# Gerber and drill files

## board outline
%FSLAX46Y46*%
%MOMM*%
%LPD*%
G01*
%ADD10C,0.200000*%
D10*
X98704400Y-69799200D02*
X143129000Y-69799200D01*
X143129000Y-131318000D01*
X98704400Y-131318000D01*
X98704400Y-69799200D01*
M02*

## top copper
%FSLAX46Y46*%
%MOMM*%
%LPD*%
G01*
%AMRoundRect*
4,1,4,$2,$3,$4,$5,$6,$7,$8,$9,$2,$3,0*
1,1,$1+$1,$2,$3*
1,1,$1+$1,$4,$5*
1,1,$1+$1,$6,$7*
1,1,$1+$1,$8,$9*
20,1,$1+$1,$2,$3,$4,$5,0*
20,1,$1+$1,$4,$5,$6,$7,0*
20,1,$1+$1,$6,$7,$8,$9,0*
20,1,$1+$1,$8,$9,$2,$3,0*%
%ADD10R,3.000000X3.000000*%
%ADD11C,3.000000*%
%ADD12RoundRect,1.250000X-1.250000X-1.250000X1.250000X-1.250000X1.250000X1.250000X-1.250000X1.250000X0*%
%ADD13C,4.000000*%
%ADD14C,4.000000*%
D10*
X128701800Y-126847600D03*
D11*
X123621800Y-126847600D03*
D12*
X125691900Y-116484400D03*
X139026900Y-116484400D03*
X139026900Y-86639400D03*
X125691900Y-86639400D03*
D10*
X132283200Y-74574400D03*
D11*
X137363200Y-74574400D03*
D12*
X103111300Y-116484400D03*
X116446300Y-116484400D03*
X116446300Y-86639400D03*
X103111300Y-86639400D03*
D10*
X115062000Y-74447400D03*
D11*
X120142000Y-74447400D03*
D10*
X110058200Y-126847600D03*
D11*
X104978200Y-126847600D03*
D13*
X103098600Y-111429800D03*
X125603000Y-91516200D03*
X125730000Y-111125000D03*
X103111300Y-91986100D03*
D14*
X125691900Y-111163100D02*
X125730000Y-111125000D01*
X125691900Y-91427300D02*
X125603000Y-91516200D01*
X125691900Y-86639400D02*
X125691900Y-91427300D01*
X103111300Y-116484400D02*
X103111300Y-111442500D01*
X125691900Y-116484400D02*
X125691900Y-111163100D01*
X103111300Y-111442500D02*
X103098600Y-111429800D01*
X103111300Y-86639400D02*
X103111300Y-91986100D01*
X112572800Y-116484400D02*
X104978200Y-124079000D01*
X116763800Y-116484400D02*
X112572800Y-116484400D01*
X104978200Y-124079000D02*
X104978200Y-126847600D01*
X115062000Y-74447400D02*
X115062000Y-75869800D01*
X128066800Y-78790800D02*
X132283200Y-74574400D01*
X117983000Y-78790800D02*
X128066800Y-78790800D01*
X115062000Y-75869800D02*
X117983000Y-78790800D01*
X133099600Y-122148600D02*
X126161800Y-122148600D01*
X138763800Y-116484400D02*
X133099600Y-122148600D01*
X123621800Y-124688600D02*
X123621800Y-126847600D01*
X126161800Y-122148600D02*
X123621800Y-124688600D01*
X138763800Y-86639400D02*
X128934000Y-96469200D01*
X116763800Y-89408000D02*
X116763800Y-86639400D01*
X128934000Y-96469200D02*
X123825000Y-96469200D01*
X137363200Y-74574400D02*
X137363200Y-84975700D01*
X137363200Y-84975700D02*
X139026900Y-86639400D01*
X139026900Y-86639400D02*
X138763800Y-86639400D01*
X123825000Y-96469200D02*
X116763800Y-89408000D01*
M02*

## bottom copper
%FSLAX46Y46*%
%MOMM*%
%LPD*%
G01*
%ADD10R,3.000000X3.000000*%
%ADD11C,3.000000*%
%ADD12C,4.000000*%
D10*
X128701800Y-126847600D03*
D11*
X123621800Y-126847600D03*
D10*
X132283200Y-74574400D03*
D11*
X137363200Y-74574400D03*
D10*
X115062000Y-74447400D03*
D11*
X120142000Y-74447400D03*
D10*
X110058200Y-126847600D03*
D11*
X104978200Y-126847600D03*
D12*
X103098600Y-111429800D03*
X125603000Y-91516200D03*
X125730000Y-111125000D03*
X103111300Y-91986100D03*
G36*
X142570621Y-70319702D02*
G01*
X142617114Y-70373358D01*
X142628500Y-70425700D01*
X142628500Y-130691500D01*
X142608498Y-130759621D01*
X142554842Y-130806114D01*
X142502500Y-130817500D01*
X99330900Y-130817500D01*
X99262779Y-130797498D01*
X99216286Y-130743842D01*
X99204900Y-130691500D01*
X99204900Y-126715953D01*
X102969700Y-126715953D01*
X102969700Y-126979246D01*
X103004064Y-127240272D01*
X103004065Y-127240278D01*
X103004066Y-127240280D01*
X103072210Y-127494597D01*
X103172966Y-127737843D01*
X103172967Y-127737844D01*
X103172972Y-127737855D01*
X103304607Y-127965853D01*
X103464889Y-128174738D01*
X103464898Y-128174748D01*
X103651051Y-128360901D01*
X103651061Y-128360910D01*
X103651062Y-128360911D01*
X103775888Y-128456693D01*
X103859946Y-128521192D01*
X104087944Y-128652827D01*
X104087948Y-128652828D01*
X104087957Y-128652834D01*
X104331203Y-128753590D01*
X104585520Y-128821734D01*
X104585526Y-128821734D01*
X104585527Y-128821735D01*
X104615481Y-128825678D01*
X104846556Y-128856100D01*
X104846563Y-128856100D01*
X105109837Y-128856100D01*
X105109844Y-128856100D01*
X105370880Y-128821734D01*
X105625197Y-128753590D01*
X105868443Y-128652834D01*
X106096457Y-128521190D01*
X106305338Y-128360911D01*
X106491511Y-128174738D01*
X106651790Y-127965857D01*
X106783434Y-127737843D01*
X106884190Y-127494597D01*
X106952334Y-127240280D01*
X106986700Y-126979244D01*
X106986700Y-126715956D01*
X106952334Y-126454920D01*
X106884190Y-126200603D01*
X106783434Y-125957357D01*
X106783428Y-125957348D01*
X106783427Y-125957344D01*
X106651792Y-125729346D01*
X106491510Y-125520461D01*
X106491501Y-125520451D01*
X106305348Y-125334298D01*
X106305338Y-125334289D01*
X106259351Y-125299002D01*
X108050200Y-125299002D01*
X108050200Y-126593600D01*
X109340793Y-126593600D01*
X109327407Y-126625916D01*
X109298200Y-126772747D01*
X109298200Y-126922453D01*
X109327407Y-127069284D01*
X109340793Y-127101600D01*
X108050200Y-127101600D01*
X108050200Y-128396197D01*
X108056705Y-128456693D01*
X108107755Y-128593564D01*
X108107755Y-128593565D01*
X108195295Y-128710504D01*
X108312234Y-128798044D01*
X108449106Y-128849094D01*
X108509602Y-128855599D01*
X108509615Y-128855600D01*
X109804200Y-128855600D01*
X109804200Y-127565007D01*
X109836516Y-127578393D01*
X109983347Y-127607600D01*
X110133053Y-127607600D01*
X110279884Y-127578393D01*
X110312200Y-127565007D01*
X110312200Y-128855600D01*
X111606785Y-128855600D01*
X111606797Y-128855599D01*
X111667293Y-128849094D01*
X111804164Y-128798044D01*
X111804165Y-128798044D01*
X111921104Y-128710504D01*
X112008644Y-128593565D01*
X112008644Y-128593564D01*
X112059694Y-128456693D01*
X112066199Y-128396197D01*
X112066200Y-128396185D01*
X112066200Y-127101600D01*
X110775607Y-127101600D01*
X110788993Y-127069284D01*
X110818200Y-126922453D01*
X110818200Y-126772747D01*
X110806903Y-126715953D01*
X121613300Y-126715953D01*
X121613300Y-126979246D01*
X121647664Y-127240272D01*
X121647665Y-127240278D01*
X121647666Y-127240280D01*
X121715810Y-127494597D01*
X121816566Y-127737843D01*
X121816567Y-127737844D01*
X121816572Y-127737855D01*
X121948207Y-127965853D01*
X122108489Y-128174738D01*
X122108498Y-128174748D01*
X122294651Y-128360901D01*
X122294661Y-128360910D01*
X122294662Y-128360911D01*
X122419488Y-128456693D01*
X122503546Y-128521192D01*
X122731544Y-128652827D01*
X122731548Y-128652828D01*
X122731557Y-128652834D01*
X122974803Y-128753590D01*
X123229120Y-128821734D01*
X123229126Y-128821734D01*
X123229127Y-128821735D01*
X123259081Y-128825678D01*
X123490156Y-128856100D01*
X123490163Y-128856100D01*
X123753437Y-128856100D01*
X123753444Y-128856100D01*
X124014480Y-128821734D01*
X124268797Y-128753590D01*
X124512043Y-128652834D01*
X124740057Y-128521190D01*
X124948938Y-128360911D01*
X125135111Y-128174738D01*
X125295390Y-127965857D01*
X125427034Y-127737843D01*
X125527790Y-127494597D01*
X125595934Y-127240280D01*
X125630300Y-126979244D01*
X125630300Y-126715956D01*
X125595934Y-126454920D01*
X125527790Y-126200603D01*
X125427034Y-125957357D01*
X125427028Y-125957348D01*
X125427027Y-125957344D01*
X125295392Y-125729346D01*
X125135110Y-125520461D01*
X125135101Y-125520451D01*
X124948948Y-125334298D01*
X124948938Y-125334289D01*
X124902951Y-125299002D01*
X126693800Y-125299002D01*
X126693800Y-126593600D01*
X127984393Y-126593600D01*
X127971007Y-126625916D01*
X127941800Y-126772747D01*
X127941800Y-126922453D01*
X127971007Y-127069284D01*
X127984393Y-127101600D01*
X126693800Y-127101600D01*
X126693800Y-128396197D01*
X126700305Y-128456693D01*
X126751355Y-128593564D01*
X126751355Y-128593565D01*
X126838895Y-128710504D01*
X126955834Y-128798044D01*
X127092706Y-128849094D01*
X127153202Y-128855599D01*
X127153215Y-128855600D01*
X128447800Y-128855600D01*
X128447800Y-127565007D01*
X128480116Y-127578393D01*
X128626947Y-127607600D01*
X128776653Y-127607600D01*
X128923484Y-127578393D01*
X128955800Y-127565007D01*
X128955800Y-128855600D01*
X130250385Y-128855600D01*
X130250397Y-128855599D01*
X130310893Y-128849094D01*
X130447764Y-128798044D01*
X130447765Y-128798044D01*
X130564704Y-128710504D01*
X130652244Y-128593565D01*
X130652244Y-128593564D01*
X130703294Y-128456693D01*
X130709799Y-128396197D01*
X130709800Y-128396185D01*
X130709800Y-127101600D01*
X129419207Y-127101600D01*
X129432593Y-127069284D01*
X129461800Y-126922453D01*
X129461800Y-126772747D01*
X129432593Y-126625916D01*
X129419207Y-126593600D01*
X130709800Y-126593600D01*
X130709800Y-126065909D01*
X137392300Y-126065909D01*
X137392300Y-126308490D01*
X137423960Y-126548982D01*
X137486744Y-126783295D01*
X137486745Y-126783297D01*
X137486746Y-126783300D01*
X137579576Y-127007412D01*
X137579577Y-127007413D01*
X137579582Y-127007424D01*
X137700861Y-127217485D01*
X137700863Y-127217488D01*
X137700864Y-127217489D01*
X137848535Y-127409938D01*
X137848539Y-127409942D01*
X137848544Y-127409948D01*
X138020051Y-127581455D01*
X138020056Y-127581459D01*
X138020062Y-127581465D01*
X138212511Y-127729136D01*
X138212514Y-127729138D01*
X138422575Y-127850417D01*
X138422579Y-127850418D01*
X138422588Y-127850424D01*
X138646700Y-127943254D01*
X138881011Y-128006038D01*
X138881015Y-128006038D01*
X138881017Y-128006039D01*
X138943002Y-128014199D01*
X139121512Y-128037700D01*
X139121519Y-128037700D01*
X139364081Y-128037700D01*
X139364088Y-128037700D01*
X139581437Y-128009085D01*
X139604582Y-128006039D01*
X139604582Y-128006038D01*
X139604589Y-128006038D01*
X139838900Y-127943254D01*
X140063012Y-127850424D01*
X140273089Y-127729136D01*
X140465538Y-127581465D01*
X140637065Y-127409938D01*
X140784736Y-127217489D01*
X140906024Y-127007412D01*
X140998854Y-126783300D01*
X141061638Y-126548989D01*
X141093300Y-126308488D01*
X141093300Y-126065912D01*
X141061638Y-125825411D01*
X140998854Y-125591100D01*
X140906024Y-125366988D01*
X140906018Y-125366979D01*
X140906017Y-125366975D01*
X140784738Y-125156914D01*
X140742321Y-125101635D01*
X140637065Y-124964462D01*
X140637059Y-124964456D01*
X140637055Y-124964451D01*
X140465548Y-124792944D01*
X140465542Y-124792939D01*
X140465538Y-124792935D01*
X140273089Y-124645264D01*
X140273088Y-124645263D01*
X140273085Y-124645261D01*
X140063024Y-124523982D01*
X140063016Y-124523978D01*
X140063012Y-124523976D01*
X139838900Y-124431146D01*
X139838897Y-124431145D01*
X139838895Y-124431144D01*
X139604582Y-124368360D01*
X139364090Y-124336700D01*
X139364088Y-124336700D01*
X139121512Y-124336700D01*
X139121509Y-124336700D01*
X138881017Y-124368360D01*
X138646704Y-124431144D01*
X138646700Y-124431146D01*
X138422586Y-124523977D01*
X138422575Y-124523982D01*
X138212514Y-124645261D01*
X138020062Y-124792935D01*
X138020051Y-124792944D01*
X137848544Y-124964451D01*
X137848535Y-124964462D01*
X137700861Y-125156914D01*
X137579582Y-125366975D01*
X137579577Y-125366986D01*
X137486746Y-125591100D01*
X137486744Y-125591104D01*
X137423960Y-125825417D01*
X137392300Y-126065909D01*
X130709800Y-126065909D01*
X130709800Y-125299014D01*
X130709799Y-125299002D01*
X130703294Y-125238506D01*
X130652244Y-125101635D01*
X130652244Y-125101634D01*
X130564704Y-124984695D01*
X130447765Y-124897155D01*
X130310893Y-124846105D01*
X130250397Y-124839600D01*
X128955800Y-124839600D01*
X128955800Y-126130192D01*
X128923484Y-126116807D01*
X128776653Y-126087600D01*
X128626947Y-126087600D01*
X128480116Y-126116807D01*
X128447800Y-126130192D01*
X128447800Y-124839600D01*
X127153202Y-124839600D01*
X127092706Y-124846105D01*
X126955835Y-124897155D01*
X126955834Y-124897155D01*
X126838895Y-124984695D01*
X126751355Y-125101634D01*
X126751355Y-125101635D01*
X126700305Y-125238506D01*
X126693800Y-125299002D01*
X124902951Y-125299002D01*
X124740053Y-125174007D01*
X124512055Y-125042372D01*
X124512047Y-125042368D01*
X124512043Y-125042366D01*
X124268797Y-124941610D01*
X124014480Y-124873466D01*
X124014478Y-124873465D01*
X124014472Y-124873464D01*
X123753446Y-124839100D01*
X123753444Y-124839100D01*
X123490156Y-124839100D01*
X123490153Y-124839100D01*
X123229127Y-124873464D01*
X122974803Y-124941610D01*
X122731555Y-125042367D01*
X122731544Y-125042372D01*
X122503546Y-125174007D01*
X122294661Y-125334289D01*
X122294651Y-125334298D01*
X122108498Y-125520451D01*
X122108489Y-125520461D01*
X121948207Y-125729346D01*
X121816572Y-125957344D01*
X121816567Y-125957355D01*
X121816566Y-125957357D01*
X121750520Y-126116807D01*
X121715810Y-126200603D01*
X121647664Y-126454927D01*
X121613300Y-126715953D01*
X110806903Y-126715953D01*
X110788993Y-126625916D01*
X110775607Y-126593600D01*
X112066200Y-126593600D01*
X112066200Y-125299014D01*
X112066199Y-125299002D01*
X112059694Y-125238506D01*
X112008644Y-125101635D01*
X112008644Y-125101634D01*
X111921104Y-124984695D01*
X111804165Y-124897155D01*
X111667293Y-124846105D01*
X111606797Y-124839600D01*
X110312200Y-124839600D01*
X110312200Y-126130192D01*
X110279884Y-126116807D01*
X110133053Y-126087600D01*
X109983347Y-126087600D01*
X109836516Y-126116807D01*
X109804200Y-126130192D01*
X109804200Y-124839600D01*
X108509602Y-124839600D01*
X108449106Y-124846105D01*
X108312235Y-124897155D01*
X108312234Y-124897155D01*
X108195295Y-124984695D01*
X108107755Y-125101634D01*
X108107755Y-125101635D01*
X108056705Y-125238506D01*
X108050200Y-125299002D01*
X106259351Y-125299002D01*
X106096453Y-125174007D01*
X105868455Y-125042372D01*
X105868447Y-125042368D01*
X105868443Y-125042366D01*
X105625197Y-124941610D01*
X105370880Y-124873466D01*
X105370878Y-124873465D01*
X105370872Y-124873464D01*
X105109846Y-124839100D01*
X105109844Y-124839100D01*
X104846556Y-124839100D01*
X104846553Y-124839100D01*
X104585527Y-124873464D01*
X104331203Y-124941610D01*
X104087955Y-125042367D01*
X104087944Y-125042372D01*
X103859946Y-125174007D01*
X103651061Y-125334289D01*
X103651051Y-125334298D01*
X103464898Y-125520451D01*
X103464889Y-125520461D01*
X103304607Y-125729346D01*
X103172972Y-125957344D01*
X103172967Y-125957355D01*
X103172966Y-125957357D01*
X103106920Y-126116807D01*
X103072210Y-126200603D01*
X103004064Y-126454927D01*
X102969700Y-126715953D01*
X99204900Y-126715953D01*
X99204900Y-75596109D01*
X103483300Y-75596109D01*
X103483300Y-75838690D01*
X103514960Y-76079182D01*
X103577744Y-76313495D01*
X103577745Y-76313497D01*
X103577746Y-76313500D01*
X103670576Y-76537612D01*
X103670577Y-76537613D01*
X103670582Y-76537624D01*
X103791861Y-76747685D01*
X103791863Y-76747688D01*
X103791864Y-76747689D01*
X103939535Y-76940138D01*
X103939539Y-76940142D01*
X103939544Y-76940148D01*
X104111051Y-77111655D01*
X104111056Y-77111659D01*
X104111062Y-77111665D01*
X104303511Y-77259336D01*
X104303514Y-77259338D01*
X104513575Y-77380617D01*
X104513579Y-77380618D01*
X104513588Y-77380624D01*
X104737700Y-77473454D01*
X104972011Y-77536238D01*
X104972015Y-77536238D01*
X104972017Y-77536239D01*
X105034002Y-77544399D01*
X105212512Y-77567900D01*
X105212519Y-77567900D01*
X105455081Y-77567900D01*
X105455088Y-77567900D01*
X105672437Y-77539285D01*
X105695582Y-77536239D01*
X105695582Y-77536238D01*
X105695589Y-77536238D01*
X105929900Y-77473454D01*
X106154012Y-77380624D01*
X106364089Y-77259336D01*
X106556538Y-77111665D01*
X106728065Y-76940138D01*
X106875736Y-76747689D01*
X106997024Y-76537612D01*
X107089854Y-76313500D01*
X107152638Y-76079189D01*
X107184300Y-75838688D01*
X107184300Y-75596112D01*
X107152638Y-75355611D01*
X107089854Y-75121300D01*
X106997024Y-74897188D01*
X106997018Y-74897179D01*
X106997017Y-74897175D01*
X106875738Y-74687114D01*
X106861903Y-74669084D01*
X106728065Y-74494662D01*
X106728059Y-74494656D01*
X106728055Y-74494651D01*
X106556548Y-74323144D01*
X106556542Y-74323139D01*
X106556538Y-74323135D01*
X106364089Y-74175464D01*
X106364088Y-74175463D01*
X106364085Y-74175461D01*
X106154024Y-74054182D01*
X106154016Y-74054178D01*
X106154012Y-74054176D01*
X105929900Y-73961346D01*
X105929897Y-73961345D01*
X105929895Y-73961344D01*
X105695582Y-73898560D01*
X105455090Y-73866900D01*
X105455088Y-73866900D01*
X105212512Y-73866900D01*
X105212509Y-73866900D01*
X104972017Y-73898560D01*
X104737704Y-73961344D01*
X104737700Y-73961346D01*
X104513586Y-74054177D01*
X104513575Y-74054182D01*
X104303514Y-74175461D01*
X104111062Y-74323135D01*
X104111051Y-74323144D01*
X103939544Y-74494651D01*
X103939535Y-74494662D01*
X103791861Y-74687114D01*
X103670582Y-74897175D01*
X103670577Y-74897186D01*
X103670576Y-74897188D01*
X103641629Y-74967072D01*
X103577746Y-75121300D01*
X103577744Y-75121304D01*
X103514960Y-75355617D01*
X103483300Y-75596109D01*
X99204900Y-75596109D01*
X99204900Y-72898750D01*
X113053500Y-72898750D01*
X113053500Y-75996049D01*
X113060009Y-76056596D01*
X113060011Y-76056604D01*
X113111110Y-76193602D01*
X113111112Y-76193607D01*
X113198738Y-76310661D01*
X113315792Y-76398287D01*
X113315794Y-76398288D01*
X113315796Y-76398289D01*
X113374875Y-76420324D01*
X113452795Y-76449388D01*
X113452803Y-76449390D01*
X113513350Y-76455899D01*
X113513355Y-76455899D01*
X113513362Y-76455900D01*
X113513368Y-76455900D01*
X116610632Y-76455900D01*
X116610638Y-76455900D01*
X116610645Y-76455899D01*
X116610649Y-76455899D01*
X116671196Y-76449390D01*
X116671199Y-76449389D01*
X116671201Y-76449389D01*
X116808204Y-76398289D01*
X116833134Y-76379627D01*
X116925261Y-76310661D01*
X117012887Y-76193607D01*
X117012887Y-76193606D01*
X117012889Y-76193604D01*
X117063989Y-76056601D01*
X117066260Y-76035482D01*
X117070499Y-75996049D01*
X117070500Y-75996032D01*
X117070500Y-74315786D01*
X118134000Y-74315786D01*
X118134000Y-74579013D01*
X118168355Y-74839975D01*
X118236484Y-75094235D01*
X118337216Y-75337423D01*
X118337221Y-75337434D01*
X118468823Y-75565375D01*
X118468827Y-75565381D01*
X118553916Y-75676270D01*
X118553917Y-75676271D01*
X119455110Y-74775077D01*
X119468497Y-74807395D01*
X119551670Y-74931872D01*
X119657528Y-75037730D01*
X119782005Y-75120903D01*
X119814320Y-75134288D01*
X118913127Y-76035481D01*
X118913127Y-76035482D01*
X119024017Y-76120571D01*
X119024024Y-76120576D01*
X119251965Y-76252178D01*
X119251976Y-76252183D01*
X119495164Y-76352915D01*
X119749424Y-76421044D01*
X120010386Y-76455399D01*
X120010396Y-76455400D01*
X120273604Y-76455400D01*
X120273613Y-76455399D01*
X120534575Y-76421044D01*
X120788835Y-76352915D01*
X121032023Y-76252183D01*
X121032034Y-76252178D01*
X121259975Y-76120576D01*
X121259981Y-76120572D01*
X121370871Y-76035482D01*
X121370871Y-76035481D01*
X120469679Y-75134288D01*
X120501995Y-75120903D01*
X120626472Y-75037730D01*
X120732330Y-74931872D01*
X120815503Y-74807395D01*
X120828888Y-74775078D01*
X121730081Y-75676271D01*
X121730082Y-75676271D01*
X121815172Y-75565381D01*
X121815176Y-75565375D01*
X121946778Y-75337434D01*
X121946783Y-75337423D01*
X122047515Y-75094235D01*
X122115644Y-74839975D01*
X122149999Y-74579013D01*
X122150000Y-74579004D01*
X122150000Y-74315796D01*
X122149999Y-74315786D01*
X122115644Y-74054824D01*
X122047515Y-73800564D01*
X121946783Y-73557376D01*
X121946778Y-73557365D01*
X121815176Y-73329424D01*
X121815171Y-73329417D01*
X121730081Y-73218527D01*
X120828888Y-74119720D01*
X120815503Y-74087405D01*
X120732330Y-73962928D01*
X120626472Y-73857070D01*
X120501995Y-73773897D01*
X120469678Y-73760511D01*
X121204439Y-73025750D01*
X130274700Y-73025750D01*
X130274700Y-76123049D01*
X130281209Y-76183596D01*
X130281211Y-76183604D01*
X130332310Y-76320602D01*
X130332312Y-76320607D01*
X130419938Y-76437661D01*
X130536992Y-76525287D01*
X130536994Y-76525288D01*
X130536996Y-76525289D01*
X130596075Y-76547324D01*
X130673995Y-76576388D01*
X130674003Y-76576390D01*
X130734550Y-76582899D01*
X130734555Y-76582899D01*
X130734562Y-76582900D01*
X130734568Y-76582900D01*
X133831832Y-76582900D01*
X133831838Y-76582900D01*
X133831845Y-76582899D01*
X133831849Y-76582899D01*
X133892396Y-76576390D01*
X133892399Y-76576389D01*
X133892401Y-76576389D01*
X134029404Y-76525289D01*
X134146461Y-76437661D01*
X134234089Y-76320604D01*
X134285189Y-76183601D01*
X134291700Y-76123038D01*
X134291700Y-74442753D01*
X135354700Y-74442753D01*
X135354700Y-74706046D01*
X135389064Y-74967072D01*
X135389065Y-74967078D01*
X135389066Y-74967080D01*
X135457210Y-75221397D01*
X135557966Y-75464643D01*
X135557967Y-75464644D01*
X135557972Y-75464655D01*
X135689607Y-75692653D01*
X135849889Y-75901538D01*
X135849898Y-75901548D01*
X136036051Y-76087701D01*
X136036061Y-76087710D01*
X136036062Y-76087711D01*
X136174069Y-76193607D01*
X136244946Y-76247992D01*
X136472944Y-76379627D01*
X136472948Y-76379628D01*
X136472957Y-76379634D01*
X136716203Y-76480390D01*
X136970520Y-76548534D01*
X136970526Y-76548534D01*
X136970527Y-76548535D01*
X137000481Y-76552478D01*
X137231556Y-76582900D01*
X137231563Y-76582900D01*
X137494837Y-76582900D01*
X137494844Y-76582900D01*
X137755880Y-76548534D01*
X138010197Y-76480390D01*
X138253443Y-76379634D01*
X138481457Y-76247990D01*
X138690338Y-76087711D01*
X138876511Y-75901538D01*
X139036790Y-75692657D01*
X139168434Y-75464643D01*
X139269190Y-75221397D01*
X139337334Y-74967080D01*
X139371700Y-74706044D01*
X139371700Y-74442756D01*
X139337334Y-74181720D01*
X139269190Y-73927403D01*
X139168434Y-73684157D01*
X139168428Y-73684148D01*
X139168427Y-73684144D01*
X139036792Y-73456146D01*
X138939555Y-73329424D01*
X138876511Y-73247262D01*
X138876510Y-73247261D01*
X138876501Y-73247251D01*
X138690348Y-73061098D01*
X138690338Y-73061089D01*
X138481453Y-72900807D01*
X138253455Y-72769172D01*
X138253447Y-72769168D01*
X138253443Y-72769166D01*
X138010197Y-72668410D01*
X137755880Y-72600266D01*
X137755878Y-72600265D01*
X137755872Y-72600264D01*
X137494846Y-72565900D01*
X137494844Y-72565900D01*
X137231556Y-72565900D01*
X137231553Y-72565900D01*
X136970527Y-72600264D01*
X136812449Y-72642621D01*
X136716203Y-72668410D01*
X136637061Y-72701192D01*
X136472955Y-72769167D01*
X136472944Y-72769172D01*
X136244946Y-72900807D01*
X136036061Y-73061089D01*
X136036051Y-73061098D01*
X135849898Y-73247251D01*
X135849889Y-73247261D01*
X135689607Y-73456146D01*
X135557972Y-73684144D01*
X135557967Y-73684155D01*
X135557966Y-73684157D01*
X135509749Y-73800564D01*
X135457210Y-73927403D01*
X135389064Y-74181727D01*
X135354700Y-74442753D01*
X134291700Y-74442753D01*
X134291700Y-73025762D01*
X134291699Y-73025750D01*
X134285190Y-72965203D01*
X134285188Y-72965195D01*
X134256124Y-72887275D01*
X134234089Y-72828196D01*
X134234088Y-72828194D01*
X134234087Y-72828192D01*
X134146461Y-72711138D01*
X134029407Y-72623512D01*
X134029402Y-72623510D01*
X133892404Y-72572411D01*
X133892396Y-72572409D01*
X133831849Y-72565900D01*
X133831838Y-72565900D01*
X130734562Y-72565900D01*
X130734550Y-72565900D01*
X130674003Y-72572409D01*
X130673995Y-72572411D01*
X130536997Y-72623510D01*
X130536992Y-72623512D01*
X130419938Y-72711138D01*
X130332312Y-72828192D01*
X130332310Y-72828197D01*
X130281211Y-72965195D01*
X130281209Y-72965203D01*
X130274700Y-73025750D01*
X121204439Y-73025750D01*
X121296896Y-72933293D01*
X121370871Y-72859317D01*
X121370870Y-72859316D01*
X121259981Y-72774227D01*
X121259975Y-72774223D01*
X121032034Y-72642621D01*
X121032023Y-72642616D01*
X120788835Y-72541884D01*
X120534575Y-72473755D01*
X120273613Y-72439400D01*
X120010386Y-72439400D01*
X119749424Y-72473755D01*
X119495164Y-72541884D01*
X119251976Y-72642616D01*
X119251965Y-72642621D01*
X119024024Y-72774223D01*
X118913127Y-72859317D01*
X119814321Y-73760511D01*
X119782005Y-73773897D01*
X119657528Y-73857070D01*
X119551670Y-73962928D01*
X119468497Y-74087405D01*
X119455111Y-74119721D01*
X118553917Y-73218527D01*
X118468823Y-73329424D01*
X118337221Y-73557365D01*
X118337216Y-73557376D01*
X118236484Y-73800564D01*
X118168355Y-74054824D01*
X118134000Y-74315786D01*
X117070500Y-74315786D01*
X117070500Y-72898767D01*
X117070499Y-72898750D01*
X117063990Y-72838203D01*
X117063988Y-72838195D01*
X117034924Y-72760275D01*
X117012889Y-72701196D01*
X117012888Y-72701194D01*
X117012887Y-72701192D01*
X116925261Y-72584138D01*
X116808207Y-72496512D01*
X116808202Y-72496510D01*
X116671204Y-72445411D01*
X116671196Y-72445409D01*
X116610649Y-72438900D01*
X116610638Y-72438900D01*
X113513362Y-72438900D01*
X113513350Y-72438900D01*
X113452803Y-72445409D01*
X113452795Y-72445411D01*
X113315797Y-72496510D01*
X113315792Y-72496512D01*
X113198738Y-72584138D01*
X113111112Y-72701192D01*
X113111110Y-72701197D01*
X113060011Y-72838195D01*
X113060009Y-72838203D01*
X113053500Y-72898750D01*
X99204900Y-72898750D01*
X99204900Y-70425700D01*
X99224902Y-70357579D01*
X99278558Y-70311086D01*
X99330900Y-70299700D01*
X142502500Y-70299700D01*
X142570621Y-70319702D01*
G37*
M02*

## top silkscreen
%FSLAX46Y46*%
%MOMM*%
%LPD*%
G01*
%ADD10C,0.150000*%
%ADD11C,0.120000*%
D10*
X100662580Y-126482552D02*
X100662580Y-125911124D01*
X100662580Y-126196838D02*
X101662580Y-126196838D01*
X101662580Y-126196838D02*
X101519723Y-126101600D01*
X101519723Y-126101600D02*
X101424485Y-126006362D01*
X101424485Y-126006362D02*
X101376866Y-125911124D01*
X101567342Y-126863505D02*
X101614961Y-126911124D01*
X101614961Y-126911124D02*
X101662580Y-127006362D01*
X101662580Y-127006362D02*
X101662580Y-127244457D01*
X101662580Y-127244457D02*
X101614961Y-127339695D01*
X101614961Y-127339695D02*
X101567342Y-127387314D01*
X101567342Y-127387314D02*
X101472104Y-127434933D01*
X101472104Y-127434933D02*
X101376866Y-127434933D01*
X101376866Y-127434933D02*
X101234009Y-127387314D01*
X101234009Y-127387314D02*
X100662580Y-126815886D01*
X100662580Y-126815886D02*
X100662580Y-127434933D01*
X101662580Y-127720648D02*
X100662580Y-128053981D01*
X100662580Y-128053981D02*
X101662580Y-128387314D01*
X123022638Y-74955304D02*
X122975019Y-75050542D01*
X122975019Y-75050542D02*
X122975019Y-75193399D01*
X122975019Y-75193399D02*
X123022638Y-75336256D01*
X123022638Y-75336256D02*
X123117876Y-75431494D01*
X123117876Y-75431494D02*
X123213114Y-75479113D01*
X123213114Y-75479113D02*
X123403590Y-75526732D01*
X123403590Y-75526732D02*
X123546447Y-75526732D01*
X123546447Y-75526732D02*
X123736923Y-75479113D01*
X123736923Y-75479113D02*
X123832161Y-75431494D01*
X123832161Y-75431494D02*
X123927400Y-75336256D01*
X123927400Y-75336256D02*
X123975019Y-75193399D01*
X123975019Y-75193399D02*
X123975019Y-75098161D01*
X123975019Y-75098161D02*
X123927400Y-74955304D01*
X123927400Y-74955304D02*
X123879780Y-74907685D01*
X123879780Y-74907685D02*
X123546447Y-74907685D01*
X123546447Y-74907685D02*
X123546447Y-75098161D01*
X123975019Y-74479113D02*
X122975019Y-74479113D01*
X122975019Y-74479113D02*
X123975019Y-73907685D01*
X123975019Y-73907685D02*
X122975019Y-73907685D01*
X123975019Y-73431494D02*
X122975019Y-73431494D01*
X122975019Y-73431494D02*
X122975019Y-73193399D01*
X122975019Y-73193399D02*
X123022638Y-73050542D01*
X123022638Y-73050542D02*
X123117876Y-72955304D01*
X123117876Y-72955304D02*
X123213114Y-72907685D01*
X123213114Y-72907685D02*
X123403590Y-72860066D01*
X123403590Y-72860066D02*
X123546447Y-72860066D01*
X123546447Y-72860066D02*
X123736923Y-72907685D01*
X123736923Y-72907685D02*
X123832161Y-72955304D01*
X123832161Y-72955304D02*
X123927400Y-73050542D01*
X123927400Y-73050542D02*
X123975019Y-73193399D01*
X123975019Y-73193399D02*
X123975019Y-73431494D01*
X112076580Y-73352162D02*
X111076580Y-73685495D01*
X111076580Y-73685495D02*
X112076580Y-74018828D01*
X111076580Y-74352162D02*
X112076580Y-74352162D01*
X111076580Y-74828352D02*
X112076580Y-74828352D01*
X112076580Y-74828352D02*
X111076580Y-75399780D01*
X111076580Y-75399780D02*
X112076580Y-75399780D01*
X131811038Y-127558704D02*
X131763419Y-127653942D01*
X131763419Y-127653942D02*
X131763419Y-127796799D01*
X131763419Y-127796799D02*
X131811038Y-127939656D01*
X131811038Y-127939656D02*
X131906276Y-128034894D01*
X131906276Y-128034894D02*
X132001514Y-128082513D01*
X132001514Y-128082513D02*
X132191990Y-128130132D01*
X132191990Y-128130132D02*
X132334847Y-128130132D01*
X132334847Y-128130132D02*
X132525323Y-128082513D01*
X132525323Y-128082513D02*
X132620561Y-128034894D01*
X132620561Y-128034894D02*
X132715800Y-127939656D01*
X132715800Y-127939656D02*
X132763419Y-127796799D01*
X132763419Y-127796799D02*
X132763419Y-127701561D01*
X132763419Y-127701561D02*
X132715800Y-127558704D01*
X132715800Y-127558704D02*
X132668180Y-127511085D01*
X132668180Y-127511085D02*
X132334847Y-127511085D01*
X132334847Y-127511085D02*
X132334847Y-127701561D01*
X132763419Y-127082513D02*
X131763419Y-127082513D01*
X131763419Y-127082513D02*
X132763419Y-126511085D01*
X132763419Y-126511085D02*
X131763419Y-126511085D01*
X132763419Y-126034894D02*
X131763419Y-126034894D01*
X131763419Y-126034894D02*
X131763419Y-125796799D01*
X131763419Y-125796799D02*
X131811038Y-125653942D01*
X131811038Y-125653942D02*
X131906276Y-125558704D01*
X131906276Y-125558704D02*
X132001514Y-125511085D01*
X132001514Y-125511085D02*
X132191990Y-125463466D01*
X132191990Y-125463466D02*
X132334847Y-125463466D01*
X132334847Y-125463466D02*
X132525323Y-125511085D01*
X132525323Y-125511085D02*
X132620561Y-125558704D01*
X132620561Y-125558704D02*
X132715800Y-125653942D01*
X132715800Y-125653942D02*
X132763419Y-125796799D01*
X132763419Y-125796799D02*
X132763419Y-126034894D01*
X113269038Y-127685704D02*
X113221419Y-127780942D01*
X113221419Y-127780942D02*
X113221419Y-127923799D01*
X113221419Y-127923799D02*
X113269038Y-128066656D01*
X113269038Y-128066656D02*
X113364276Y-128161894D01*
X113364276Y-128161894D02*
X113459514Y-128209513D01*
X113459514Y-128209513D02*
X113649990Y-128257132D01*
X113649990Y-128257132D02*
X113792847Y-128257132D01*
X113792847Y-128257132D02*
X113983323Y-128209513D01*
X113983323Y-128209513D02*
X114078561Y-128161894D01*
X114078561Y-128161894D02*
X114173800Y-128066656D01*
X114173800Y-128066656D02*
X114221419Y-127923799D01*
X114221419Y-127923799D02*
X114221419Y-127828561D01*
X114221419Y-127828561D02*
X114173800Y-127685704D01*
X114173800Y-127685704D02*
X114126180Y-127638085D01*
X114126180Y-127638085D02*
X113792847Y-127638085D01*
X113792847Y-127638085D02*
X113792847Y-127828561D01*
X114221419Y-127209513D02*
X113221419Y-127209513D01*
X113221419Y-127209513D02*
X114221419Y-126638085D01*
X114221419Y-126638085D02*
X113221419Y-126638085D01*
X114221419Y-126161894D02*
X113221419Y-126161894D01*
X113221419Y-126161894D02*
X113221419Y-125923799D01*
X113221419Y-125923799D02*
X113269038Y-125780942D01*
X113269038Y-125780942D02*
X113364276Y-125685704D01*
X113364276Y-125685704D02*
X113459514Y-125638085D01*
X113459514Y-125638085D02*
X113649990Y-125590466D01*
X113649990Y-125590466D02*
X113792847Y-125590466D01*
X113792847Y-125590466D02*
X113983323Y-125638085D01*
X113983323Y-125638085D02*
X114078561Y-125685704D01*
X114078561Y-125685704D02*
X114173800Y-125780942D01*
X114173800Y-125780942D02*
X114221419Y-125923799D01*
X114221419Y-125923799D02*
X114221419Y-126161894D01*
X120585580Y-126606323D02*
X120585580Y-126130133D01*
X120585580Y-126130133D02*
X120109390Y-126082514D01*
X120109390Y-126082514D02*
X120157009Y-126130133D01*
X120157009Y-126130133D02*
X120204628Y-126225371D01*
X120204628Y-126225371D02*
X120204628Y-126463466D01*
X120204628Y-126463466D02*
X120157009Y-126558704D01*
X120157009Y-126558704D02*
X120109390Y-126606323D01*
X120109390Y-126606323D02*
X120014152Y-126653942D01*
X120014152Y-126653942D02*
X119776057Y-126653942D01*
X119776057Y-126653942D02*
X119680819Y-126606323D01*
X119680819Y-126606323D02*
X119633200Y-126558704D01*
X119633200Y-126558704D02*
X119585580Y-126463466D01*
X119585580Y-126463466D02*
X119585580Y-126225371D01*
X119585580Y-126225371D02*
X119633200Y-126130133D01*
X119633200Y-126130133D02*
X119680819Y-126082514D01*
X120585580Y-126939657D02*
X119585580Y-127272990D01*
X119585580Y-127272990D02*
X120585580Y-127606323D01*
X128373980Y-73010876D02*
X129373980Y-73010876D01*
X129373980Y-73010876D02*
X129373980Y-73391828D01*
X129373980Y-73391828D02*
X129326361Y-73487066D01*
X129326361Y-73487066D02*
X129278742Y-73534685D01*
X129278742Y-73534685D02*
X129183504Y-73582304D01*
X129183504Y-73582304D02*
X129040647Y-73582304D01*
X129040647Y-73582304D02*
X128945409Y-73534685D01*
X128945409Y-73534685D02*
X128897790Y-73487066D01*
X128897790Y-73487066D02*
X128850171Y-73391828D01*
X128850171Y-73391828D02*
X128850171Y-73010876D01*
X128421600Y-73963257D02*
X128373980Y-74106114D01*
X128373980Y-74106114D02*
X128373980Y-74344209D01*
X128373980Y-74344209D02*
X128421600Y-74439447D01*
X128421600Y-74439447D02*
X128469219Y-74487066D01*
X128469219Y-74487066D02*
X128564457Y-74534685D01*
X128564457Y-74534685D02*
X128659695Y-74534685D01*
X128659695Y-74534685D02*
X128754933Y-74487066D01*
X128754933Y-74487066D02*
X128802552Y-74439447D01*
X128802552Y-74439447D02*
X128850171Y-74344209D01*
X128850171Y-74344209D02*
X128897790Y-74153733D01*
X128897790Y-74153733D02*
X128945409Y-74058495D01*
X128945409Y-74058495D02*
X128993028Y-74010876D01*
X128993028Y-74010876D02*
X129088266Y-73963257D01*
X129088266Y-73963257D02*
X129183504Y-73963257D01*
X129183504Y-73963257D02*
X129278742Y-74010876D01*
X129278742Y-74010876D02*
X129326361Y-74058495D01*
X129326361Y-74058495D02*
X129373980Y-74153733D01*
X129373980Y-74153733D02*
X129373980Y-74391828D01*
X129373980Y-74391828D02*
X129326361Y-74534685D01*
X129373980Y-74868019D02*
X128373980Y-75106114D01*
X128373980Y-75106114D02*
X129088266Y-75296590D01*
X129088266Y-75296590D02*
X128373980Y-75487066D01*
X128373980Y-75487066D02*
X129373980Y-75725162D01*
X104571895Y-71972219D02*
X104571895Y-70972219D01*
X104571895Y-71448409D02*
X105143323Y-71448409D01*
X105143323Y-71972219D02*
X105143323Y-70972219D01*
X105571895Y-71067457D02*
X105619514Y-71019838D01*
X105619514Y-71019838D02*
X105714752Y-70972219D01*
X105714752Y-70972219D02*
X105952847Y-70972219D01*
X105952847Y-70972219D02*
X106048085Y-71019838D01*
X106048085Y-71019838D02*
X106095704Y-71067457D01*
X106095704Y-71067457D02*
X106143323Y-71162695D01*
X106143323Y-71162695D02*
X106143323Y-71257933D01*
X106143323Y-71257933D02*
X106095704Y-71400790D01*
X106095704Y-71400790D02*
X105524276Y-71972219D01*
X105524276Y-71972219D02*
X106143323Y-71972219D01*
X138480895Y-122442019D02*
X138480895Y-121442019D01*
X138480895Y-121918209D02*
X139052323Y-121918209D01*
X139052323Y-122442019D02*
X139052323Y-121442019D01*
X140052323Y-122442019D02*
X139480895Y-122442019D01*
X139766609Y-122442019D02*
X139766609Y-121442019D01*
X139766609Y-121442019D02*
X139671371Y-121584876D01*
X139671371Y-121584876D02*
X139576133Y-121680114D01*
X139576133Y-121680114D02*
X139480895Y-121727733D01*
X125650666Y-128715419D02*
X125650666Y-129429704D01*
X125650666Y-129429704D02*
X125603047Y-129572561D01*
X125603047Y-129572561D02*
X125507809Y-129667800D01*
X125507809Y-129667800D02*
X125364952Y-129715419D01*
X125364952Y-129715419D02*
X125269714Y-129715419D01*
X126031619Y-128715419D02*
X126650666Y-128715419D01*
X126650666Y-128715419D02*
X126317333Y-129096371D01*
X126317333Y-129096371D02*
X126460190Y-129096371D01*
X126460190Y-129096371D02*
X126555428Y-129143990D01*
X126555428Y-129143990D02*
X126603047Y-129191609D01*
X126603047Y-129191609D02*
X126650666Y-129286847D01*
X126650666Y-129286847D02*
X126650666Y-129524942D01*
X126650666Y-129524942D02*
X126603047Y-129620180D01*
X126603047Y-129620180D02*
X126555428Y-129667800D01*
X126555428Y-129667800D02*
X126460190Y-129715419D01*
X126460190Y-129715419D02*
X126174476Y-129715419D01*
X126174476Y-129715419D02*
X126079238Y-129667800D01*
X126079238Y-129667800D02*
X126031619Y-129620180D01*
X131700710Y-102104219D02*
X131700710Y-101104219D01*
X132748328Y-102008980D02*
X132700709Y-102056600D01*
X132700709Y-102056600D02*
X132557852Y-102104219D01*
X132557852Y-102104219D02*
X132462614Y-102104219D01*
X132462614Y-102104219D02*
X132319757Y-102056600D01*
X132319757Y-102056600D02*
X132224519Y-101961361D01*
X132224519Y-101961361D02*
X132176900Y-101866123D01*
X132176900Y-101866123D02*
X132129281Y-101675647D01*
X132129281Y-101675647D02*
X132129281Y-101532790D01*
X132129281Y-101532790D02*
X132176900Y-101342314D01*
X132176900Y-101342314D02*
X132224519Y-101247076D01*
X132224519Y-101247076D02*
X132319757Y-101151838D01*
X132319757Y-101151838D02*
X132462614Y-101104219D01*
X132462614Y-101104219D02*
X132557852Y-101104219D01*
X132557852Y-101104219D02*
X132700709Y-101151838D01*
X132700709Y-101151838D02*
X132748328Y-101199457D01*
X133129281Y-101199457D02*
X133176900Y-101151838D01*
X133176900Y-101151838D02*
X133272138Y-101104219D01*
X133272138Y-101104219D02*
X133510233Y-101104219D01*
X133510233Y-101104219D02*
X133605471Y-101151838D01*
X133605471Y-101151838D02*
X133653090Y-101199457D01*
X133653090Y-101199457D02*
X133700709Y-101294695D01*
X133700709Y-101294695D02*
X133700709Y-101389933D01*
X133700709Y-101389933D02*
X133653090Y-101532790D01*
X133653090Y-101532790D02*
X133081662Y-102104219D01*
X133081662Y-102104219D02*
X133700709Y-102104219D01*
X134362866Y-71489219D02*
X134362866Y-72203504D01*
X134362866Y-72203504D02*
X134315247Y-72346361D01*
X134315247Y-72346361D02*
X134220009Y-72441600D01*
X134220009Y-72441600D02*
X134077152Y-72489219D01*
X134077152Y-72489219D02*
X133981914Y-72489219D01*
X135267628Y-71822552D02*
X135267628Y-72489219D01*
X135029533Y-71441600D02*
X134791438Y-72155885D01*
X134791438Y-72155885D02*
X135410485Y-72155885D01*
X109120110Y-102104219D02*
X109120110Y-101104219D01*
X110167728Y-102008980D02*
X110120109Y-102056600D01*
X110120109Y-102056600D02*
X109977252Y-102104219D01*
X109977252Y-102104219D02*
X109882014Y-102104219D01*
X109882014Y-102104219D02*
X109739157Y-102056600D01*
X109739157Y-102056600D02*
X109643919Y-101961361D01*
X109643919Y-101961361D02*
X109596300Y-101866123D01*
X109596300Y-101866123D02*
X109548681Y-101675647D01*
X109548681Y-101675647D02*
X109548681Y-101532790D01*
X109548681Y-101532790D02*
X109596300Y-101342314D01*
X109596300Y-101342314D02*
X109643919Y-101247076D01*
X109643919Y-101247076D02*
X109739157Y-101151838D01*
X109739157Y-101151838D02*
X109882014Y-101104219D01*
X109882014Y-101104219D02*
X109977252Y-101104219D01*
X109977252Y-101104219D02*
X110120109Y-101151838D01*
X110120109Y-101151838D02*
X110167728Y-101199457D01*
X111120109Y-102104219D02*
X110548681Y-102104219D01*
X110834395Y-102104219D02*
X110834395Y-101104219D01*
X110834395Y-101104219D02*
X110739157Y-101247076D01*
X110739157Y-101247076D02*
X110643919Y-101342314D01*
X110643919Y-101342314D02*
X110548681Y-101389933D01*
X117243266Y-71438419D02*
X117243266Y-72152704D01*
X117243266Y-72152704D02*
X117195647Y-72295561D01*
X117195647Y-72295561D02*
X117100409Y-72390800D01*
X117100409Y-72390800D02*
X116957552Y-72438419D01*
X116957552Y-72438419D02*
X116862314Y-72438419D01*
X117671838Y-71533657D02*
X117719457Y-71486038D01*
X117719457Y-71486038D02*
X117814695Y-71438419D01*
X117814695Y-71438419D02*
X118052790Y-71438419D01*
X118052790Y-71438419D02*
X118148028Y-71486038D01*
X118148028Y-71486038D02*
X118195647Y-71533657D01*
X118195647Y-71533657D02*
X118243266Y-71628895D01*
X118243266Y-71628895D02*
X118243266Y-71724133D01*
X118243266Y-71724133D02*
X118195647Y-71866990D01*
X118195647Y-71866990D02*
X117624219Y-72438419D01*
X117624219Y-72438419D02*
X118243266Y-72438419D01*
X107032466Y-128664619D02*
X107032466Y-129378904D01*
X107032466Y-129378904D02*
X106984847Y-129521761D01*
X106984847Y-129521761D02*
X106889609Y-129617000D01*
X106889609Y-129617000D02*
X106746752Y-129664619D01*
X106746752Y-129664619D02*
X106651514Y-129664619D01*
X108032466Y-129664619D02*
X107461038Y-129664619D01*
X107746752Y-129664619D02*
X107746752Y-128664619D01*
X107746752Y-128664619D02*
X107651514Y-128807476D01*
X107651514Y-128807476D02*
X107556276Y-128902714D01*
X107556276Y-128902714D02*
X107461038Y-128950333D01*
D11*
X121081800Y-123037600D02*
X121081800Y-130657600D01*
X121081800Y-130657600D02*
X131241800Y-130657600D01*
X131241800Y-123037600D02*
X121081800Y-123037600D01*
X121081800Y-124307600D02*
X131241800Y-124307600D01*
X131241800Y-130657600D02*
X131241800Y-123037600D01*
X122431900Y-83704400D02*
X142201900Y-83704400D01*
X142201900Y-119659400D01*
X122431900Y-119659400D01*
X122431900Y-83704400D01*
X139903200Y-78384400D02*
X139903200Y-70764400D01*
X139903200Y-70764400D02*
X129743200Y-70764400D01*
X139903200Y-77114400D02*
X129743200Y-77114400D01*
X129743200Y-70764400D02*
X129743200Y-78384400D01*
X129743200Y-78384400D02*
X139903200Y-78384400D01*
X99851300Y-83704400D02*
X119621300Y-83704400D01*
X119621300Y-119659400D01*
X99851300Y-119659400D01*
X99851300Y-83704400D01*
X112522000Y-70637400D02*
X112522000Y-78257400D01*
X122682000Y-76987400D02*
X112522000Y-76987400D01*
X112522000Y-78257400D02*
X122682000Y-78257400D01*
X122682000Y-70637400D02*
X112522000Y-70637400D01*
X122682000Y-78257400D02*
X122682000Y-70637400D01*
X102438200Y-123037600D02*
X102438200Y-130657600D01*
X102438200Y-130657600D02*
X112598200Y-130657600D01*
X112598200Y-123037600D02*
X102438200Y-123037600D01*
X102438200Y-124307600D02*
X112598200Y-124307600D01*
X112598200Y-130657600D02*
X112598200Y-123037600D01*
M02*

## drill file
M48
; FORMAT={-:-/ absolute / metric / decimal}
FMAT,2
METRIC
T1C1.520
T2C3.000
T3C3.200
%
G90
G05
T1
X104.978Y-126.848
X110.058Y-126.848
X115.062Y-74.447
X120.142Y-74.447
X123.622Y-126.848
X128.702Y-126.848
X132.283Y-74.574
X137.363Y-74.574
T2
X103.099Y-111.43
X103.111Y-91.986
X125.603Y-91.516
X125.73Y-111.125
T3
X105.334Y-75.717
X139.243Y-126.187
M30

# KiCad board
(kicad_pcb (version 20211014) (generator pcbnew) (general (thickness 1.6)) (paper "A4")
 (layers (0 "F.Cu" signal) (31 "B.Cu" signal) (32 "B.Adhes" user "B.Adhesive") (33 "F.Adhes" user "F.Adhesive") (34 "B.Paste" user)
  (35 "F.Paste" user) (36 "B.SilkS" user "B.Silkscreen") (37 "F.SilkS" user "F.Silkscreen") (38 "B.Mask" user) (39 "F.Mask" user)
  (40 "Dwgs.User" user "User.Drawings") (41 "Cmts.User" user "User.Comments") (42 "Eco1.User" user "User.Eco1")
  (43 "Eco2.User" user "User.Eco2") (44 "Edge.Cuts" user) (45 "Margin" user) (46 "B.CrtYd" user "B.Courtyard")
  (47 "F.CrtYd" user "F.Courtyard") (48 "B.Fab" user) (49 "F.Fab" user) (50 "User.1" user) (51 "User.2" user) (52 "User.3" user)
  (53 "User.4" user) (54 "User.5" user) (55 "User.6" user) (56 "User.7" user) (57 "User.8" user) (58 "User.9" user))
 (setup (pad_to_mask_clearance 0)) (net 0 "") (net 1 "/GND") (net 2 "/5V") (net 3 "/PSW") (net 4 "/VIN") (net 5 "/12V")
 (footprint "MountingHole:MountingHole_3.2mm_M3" (layer "F.Cu") (at 105.3338 75.7174)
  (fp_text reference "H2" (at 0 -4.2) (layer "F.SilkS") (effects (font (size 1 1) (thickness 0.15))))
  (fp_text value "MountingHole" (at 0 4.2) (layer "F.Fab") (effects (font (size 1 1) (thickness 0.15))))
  (pad "" np_thru_hole circle (at 0 0) (size 3.2 3.2) (drill 3.2) (layers *.Cu *.Mask)))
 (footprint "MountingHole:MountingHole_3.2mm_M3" (layer "F.Cu") (at 139.2428 126.1872)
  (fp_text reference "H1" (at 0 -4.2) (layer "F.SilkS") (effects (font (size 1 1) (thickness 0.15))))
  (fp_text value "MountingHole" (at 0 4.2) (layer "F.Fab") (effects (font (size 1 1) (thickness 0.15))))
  (pad "" np_thru_hole circle (at 0 0) (size 3.2 3.2) (drill 3.2) (layers *.Cu *.Mask)))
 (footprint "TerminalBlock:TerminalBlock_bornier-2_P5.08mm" (layer "F.Cu") (at 128.7018 126.8476 180)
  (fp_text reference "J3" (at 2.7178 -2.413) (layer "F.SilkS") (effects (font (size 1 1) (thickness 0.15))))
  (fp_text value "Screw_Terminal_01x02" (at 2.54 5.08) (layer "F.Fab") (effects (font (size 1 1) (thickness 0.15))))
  (fp_line (start 7.62 3.81) (end 7.62 -3.81) (layer "F.SilkS") (width 0.12))
  (fp_line (start 7.62 -3.81) (end -2.54 -3.81) (layer "F.SilkS") (width 0.12))
  (fp_line (start -2.54 3.81) (end 7.62 3.81) (layer "F.SilkS") (width 0.12))
  (fp_line (start 7.62 2.54) (end -2.54 2.54) (layer "F.SilkS") (width 0.12))
  (fp_line (start -2.54 -3.81) (end -2.54 3.81) (layer "F.SilkS") (width 0.12))
  (pad "1" thru_hole rect (at 0 0 180) (size 3 3) (drill 1.52) (layers *.Cu *.Mask) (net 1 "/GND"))
  (pad "2" thru_hole circle (at 5.08 0 180) (size 3 3) (drill 1.52) (layers *.Cu *.Mask) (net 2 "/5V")))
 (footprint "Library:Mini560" (layer "F.Cu") (at 123.1519 86.6394)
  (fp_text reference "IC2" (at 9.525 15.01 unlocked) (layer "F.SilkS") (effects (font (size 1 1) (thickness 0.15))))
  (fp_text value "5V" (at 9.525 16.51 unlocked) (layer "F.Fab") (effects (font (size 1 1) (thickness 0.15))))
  (fp_rect (start -0.72 -2.935) (end 19.05 33.02) (layer "F.SilkS") (width 0.12) (fill none))
  (pad "1" smd roundrect (at 2.54 29.845) (size 5 5) (layers "F.Cu" "F.Paste" "F.Mask") (roundrect_rratio 0.25) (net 1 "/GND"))
  (pad "2" smd roundrect (at 15.875 29.845) (size 5 5) (layers "F.Cu" "F.Paste" "F.Mask") (roundrect_rratio 0.25) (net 2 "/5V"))
  (pad "3" smd roundrect (at 15.875 0) (size 5 5) (layers "F.Cu" "F.Paste" "F.Mask") (roundrect_rratio 0.25) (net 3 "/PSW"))
  (pad "4" smd roundrect (at 2.54 0) (size 5 5) (layers "F.Cu" "F.Paste" "F.Mask") (roundrect_rratio 0.25) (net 1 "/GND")))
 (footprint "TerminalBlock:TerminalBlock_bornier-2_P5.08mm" (layer "F.Cu") (at 132.2832 74.5744)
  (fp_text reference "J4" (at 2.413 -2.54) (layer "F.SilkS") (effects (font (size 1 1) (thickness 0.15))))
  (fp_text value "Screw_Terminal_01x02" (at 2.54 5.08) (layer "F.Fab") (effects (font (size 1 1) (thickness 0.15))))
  (fp_line (start 7.62 3.81) (end 7.62 -3.81) (layer "F.SilkS") (width 0.12))
  (fp_line (start 7.62 -3.81) (end -2.54 -3.81) (layer "F.SilkS") (width 0.12))
  (fp_line (start 7.62 2.54) (end -2.54 2.54) (layer "F.SilkS") (width 0.12))
  (fp_line (start -2.54 -3.81) (end -2.54 3.81) (layer "F.SilkS") (width 0.12))
  (fp_line (start -2.54 3.81) (end 7.62 3.81) (layer "F.SilkS") (width 0.12))
  (pad "1" thru_hole rect (at 0 0) (size 3 3) (drill 1.52) (layers *.Cu *.Mask) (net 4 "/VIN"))
  (pad "2" thru_hole circle (at 5.08 0) (size 3 3) (drill 1.52) (layers *.Cu *.Mask) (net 3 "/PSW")))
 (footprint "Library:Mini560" (layer "F.Cu") (at 100.5713 86.6394)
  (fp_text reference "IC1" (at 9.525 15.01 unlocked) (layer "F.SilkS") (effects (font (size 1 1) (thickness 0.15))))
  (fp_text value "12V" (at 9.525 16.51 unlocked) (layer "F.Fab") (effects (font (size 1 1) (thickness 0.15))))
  (fp_rect (start -0.72 -2.935) (end 19.05 33.02) (layer "F.SilkS") (width 0.12) (fill none))
  (pad "1" smd roundrect (at 2.54 29.845) (size 5 5) (layers "F.Cu" "F.Paste" "F.Mask") (roundrect_rratio 0.25) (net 1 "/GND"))
  (pad "2" smd roundrect (at 15.875 29.845) (size 5 5) (layers "F.Cu" "F.Paste" "F.Mask") (roundrect_rratio 0.25) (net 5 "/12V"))
  (pad "3" smd roundrect (at 15.875 0) (size 5 5) (layers "F.Cu" "F.Paste" "F.Mask") (roundrect_rratio 0.25) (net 3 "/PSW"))
  (pad "4" smd roundrect (at 2.54 0) (size 5 5) (layers "F.Cu" "F.Paste" "F.Mask") (roundrect_rratio 0.25) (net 1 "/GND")))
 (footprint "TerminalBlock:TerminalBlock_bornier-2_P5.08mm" (layer "F.Cu") (at 115.062 74.4474)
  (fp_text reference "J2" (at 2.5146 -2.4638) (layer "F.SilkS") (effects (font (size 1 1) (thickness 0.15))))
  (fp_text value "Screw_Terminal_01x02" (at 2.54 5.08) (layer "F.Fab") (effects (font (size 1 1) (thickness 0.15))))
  (fp_line (start -2.54 -3.81) (end -2.54 3.81) (layer "F.SilkS") (width 0.12))
  (fp_line (start 7.62 2.54) (end -2.54 2.54) (layer "F.SilkS") (width 0.12))
  (fp_line (start -2.54 3.81) (end 7.62 3.81) (layer "F.SilkS") (width 0.12))
  (fp_line (start 7.62 -3.81) (end -2.54 -3.81) (layer "F.SilkS") (width 0.12))
  (fp_line (start 7.62 3.81) (end 7.62 -3.81) (layer "F.SilkS") (width 0.12))
  (pad "1" thru_hole rect (at 0 0) (size 3 3) (drill 1.52) (layers *.Cu *.Mask) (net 4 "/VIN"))
  (pad "2" thru_hole circle (at 5.08 0) (size 3 3) (drill 1.52) (layers *.Cu *.Mask) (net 1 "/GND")))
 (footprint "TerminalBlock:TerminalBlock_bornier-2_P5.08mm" (layer "F.Cu") (at 110.0582 126.8476 180)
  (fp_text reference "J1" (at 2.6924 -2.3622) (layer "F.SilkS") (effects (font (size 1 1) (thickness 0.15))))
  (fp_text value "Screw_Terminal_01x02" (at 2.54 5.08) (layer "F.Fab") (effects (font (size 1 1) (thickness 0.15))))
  (fp_line (start 7.62 3.81) (end 7.62 -3.81) (layer "F.SilkS") (width 0.12))
  (fp_line (start 7.62 -3.81) (end -2.54 -3.81) (layer "F.SilkS") (width 0.12))
  (fp_line (start -2.54 3.81) (end 7.62 3.81) (layer "F.SilkS") (width 0.12))
  (fp_line (start 7.62 2.54) (end -2.54 2.54) (layer "F.SilkS") (width 0.12))
  (fp_line (start -2.54 -3.81) (end -2.54 3.81) (layer "F.SilkS") (width 0.12))
  (pad "1" thru_hole rect (at 0 0 180) (size 3 3) (drill 1.52) (layers *.Cu *.Mask) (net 1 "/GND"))
  (pad "2" thru_hole circle (at 5.08 0 180) (size 3 3) (drill 1.52) (layers *.Cu *.Mask) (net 5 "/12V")))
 (gr_rect (start 143.129 131.318) (end 98.7044 69.7992) (layer "Edge.Cuts") (width 0.2) (fill none))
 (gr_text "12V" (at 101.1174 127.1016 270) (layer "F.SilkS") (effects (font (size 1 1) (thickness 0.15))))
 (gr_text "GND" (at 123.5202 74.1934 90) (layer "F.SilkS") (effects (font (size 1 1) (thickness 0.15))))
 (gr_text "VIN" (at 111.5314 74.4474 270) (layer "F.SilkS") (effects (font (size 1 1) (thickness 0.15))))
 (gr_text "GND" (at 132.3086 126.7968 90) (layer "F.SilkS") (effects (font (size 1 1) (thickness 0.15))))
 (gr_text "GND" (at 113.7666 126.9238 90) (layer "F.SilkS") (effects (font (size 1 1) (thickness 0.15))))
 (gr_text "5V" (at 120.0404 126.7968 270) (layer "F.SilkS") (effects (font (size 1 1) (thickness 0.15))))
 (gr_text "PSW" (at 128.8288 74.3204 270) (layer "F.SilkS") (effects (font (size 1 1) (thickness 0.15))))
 (segment (start 125.6919 111.1631) (end 125.73 111.125) (width 4) (layer "F.Cu") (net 1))
 (segment (start 125.6919 91.4273) (end 125.603 91.5162) (width 4) (layer "F.Cu") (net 1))
 (segment (start 125.6919 86.6394) (end 125.6919 91.4273) (width 4) (layer "F.Cu") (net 1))
 (segment (start 103.1113 116.4844) (end 103.1113 111.4425) (width 4) (layer "F.Cu") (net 1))
 (segment (start 125.6919 116.4844) (end 125.6919 111.1631) (width 4) (layer "F.Cu") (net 1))
 (segment (start 103.1113 111.4425) (end 103.0986 111.4298) (width 4) (layer "F.Cu") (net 1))
 (segment (start 103.1113 86.6394) (end 103.1113 91.9861) (width 4) (layer "F.Cu") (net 1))
 (via (at 103.0986 111.4298) (size 4) (drill 3) (layers "F.Cu" "B.Cu") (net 1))
 (via (at 125.603 91.5162) (size 4) (drill 3) (layers "F.Cu" "B.Cu") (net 1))
 (via (at 125.73 111.125) (size 4) (drill 3) (layers "F.Cu" "B.Cu") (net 1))
 (via (at 103.1113 91.9861) (size 4) (drill 3) (layers "F.Cu" "B.Cu") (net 1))
 (segment (start 112.5728 116.4844) (end 104.9782 124.079) (width 4) (layer "F.Cu") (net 5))
 (segment (start 116.7638 116.4844) (end 112.5728 116.4844) (width 4) (layer "F.Cu") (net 5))
 (segment (start 104.9782 124.079) (end 104.9782 126.8476) (width 4) (layer "F.Cu") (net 5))
 (segment (start 115.062 74.4474) (end 115.062 75.8698) (width 4) (layer "F.Cu") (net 4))
 (segment (start 128.0668 78.7908) (end 132.2832 74.5744) (width 4) (layer "F.Cu") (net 4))
 (segment (start 117.983 78.7908) (end 128.0668 78.7908) (width 4) (layer "F.Cu") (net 4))
 (segment (start 115.062 75.8698) (end 117.983 78.7908) (width 4) (layer "F.Cu") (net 4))
 (segment (start 133.0996 122.1486) (end 126.1618 122.1486) (width 4) (layer "F.Cu") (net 2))
 (segment (start 138.7638 116.4844) (end 133.0996 122.1486) (width 4) (layer "F.Cu") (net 2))
 (segment (start 123.6218 124.6886) (end 123.6218 126.8476) (width 4) (layer "F.Cu") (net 2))
 (segment (start 126.1618 122.1486) (end 123.6218 124.6886) (width 4) (layer "F.Cu") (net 2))
 (segment (start 138.7638 86.6394) (end 128.934 96.4692) (width 4) (layer "F.Cu") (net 3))
 (segment (start 116.7638 89.408) (end 116.7638 86.6394) (width 4) (layer "F.Cu") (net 3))
 (segment (start 128.934 96.4692) (end 123.825 96.4692) (width 4) (layer "F.Cu") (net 3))
 (segment (start 137.3632 74.5744) (end 137.3632 84.9757) (width 4) (layer "F.Cu") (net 3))
 (segment (start 137.3632 84.9757) (end 139.0269 86.6394) (width 4) (layer "F.Cu") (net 3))
 (segment (start 139.0269 86.6394) (end 138.7638 86.6394) (width 4) (layer "F.Cu") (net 3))
 (segment (start 123.825 96.4692) (end 116.7638 89.408) (width 4) (layer "F.Cu") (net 3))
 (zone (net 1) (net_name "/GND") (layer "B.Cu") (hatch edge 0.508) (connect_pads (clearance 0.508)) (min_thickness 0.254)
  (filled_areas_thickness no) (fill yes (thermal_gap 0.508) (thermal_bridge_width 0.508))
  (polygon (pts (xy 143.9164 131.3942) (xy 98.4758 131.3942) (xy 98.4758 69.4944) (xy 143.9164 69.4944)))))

